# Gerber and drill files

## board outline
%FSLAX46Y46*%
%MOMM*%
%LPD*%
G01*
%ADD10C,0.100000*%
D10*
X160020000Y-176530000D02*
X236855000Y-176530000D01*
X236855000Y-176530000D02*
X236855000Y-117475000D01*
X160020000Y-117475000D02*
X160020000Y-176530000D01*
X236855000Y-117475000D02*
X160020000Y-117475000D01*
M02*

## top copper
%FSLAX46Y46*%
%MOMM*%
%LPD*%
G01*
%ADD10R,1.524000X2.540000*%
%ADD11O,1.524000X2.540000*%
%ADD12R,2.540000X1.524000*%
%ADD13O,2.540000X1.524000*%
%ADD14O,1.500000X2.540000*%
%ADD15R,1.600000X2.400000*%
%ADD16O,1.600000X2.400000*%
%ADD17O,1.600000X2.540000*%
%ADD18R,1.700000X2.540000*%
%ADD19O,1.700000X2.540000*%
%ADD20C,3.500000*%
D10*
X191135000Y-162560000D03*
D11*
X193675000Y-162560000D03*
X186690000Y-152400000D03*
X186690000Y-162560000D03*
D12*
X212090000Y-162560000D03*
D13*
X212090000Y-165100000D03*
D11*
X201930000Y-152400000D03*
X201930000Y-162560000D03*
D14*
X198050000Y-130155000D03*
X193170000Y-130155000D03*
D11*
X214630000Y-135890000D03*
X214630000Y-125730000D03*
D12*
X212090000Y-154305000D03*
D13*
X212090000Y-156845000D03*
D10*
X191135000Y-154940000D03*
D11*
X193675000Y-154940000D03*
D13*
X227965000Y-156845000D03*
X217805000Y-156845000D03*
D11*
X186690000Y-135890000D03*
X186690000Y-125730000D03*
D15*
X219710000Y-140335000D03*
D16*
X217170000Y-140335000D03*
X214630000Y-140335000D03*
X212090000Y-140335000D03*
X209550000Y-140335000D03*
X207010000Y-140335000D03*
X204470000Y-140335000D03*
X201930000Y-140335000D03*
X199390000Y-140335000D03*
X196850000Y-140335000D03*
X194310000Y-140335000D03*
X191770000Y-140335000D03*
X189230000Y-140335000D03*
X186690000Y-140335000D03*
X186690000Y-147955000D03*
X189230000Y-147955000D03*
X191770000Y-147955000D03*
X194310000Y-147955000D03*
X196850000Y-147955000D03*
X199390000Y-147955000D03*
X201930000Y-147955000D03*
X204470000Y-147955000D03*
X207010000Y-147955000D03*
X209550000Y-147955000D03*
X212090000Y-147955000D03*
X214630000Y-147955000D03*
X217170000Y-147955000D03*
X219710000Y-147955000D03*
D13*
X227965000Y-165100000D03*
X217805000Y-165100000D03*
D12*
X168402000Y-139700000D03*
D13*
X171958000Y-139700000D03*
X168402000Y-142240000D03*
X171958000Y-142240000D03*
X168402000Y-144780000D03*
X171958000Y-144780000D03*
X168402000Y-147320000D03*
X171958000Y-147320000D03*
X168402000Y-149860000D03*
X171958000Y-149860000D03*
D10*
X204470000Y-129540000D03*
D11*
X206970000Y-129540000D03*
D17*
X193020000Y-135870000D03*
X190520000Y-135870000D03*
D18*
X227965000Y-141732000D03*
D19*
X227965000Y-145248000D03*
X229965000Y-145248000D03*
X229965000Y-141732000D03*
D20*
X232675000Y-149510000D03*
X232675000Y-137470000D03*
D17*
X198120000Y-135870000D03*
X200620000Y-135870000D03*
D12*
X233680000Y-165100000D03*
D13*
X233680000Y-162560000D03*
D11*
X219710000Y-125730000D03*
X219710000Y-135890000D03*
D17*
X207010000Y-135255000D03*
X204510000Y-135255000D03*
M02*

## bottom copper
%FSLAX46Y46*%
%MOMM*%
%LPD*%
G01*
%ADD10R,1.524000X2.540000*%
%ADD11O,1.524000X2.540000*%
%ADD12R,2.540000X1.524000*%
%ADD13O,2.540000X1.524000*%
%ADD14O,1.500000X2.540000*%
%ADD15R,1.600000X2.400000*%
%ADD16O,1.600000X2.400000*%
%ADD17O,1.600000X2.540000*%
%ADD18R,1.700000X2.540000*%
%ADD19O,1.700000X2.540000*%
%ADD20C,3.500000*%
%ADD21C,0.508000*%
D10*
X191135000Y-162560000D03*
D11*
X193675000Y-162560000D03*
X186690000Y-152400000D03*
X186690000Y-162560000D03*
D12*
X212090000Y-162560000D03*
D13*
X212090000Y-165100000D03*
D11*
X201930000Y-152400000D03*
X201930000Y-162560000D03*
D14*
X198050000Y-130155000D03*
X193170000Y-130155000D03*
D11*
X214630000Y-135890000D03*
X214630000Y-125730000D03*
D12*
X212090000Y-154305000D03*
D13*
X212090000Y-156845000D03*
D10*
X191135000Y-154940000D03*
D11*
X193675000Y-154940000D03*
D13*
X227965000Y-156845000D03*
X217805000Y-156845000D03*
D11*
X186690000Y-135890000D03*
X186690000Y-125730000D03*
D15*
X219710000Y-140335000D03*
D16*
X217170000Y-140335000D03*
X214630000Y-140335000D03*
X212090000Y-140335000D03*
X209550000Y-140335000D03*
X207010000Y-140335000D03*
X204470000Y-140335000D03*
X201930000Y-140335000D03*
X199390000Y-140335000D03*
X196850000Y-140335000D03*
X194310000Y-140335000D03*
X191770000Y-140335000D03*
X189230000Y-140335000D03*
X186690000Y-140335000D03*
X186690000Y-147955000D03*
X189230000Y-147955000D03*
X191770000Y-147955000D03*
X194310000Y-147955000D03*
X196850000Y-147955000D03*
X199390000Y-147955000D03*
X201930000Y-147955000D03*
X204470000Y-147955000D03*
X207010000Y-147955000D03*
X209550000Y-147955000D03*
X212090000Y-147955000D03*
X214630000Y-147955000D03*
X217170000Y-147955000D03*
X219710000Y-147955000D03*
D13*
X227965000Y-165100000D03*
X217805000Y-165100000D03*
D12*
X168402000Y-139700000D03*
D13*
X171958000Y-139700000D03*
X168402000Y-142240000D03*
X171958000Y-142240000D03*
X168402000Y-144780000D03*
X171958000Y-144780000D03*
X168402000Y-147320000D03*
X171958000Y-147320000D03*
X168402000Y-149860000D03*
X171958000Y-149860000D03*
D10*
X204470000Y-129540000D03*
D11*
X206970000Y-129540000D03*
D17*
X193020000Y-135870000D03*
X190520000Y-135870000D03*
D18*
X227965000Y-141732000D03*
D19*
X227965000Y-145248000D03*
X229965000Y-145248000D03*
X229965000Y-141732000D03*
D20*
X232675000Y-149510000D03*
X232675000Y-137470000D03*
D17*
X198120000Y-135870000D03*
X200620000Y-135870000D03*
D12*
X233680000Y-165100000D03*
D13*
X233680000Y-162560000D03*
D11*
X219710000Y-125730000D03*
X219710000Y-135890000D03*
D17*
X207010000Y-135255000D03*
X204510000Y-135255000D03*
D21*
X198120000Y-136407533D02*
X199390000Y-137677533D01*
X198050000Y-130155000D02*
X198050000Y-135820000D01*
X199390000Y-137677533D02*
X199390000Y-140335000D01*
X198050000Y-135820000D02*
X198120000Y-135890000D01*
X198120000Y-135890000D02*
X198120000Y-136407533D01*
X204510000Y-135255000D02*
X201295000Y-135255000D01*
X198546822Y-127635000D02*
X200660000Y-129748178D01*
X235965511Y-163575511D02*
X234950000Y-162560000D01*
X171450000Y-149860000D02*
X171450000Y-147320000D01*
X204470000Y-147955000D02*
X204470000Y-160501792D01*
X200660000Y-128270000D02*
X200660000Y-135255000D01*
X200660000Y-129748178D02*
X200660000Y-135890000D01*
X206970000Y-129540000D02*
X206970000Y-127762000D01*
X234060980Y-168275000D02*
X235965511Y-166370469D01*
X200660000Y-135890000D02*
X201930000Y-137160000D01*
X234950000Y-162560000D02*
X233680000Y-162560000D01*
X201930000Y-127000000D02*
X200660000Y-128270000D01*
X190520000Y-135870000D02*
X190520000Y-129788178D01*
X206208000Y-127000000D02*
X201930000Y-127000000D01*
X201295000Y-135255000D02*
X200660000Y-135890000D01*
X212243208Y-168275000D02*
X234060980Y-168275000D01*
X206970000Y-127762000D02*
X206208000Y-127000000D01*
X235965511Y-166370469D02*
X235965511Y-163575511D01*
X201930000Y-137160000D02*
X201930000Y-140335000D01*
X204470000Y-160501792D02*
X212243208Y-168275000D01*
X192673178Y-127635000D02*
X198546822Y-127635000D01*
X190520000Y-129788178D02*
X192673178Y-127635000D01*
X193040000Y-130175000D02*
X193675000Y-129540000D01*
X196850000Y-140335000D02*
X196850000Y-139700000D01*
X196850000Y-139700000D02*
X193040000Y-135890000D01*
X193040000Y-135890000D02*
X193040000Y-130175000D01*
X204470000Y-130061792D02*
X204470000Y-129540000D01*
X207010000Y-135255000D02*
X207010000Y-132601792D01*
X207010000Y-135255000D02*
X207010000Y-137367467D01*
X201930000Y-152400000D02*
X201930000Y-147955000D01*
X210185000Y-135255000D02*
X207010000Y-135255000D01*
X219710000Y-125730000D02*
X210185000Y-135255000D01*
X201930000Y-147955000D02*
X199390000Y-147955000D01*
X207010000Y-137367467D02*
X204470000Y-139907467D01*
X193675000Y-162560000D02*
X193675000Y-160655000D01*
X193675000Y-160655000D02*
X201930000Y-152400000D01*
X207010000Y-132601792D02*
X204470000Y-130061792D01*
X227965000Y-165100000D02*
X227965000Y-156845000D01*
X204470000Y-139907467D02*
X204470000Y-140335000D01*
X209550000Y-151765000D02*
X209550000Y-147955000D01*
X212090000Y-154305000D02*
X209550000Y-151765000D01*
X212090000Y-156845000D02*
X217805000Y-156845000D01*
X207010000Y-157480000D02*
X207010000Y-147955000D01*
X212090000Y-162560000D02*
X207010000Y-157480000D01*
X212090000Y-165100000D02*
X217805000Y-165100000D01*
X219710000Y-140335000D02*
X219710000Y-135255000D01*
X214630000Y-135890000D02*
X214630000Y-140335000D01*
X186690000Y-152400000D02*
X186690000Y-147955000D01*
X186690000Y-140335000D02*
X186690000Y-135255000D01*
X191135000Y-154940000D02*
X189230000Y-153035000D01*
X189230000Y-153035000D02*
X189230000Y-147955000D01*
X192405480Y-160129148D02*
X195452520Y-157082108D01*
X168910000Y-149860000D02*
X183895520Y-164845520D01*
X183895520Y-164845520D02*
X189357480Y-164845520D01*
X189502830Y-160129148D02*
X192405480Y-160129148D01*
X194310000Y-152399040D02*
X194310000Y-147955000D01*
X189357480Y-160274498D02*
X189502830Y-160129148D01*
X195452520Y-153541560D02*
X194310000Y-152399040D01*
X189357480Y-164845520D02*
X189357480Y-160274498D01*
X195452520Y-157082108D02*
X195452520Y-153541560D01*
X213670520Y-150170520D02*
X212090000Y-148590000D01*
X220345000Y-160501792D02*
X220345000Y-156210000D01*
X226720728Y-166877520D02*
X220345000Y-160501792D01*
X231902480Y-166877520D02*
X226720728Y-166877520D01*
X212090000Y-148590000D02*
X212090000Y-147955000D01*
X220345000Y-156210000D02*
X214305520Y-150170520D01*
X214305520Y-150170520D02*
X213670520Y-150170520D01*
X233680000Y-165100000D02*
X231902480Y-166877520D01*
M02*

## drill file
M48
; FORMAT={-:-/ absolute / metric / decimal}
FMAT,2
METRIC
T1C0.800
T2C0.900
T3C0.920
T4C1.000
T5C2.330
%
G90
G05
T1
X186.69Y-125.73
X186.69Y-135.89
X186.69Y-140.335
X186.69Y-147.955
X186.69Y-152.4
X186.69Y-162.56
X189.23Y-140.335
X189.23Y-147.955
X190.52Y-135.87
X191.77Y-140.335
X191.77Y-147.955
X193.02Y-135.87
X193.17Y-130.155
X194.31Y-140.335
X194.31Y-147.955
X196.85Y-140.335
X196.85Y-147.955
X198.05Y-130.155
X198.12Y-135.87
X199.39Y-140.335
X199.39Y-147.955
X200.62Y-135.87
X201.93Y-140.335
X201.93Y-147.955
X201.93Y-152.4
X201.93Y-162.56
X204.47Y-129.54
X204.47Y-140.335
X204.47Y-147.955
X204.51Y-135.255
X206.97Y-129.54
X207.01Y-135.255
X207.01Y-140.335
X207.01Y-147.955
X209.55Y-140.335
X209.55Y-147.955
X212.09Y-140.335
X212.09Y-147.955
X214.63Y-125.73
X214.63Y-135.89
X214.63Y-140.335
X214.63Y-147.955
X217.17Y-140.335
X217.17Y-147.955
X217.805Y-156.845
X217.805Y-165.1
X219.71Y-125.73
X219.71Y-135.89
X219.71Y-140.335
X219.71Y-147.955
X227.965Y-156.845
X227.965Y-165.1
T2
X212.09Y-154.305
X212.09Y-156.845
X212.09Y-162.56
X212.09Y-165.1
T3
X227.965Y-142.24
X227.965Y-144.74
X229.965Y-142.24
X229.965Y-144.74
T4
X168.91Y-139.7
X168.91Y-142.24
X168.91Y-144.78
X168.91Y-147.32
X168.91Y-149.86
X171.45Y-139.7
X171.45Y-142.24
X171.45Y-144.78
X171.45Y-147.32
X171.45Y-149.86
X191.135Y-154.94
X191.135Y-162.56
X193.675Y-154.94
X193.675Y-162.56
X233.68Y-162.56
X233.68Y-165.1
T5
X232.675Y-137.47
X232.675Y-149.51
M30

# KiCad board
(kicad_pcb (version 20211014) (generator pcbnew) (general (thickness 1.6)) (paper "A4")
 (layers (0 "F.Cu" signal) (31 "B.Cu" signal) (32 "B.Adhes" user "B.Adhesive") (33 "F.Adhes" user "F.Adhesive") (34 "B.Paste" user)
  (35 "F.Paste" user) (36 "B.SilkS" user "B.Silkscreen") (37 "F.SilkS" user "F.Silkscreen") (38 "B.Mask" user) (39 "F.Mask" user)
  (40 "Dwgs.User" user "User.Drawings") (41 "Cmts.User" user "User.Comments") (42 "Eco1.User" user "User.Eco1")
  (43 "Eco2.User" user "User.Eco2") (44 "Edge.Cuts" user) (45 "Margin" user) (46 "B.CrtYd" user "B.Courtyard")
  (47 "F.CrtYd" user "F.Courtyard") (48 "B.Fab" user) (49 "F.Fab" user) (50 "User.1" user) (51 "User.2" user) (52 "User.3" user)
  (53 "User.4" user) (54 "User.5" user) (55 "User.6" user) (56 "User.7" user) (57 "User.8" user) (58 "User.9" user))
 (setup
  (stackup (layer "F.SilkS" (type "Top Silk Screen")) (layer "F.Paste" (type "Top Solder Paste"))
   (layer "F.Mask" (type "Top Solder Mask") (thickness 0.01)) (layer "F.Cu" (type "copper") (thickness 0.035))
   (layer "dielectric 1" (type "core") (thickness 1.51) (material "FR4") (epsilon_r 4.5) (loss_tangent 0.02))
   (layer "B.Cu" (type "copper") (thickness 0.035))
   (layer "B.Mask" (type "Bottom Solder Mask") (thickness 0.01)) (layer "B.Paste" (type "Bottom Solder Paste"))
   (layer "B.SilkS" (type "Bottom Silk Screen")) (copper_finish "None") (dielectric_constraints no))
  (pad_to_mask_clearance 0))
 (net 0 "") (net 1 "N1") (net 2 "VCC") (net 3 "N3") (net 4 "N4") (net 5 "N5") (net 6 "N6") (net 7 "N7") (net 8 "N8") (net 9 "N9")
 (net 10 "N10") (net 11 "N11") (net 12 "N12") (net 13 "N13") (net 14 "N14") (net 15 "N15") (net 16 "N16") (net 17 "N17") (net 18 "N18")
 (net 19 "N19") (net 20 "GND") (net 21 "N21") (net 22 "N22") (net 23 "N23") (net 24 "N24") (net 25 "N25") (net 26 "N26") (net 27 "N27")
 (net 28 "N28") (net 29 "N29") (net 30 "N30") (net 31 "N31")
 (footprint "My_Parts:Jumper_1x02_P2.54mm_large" (layer "F.Cu") (at 191.135 162.56 90)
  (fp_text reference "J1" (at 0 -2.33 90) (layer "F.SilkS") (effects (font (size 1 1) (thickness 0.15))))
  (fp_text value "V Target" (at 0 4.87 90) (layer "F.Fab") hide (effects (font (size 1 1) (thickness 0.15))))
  (pad "1" thru_hole rect locked (at 0 0 90) (size 2.54 1.524) (drill 1) (layers *.Cu *.Mask) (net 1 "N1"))
  (pad "2" thru_hole oval locked (at 0 2.54 90) (size 2.54 1.524) (drill 1) (layers *.Cu *.Mask) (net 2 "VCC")))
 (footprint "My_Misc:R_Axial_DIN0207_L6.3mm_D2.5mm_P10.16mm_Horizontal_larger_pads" (layer "F.Cu") (at 186.69 152.4 -90)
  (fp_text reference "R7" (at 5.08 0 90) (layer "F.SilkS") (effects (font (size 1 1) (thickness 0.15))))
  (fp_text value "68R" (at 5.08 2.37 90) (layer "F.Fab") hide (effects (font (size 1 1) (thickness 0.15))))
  (pad "1" thru_hole oval (at 0 0 270) (size 2.54 1.524) (drill 0.8) (layers *.Cu *.Mask) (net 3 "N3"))
  (pad "2" thru_hole oval (at 10.16 0 270) (size 2.54 1.524) (drill 0.8) (layers *.Cu *.Mask) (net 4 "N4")))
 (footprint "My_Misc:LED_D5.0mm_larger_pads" (layer "F.Cu") (at 212.09 162.56 -90)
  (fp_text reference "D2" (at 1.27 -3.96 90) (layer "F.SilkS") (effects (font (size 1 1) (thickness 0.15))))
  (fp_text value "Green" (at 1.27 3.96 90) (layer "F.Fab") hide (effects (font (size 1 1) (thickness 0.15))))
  (pad "1" thru_hole rect locked (at 0 0 270) (size 1.524 2.54) (drill 0.9) (layers *.Cu *.Mask) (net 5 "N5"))
  (pad "2" thru_hole oval locked (at 2.54 0 270) (size 1.524 2.54) (drill 0.9) (layers *.Cu *.Mask) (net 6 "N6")))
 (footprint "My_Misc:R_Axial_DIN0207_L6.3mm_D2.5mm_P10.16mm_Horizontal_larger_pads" (layer "F.Cu") (at 201.93 152.4 -90)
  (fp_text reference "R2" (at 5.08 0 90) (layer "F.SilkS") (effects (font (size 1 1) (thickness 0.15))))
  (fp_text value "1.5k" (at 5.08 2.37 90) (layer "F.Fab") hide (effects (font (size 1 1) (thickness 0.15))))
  (pad "1" thru_hole oval (at 0 0 270) (size 2.54 1.524) (drill 0.8) (layers *.Cu *.Mask) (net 2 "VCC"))
  (pad "2" thru_hole oval (at 10.16 0 270) (size 2.54 1.524) (drill 0.8) (layers *.Cu *.Mask) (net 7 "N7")))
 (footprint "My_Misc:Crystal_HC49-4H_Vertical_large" (layer "F.Cu") (at 198.05 130.155 180)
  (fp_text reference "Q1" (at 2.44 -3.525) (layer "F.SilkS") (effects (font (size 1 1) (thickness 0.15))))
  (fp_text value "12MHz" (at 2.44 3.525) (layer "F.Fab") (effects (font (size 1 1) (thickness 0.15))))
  (pad "1" thru_hole oval locked (at 0 0 180) (size 1.5 2.54) (drill 0.8) (layers *.Cu *.Mask) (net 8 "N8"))
  (pad "2" thru_hole oval locked (at 4.88 0 180) (size 1.5 2.54) (drill 0.8) (layers *.Cu *.Mask) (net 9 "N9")))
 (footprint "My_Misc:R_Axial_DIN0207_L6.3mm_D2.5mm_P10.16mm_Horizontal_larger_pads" (layer "F.Cu") (at 214.63 135.89 90)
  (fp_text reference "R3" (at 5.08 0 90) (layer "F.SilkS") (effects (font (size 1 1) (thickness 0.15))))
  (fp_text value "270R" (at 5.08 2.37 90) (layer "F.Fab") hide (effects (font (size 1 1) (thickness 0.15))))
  (pad "1" thru_hole oval (at 0 0 90) (size 2.54 1.524) (drill 0.8) (layers *.Cu *.Mask) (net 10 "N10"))
  (pad "2" thru_hole oval (at 10.16 0 90) (size 2.54 1.524) (drill 0.8) (layers *.Cu *.Mask) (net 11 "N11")))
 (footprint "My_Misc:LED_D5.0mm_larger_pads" (layer "F.Cu") (at 212.09 154.305 -90)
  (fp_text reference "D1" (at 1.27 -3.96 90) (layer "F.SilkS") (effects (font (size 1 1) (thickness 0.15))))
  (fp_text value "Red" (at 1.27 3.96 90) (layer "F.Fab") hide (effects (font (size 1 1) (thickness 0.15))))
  (pad "1" thru_hole rect locked (at 0 0 270) (size 1.524 2.54) (drill 0.9) (layers *.Cu *.Mask) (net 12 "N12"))
  (pad "2" thru_hole oval locked (at 2.54 0 270) (size 1.524 2.54) (drill 0.9) (layers *.Cu *.Mask) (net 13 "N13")))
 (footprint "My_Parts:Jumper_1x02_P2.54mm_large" (layer "F.Cu") (at 191.135 154.94 90)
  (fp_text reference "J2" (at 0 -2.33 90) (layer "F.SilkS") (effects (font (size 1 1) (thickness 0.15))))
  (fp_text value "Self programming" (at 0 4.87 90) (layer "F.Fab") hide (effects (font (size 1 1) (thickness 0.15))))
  (pad "1" thru_hole rect locked (at 0 0 90) (size 2.54 1.524) (drill 1) (layers *.Cu *.Mask) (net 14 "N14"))
  (pad "2" thru_hole oval locked (at 0 2.54 90) (size 2.54 1.524) (drill 1) (layers *.Cu *.Mask) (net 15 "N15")))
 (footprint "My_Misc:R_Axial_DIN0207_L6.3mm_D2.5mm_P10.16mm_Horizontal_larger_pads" (layer "F.Cu") (at 227.965 156.845 180)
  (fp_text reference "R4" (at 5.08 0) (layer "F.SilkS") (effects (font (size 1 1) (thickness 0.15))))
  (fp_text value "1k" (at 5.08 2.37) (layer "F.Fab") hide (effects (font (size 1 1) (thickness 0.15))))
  (pad "1" thru_hole oval (at 0 0 180) (size 2.54 1.524) (drill 0.8) (layers *.Cu *.Mask) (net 2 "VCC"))
  (pad "2" thru_hole oval (at 10.16 0 180) (size 2.54 1.524) (drill 0.8) (layers *.Cu *.Mask) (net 13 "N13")))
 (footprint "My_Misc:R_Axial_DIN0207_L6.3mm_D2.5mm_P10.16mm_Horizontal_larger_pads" (layer "F.Cu") (at 186.69 135.89 90)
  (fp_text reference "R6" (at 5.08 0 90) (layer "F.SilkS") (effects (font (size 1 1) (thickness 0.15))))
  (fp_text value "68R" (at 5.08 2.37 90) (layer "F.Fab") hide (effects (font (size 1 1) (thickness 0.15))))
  (pad "1" thru_hole oval (at 0 0 90) (size 2.54 1.524) (drill 0.8) (layers *.Cu *.Mask) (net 7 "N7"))
  (pad "2" thru_hole oval (at 10.16 0 90) (size 2.54 1.524) (drill 0.8) (layers *.Cu *.Mask) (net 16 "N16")))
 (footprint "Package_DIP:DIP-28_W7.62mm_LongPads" (layer "F.Cu") (at 219.71 140.335 -90)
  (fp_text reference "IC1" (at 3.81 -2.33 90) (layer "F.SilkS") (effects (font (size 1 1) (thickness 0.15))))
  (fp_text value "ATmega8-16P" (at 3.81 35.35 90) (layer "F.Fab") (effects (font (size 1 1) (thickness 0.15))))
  (pad "1" thru_hole rect (at 0 0 270) (size 2.4 1.6) (drill 0.8) (layers *.Cu *.Mask) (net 15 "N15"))
  (pad "2" thru_hole oval (at 0 2.54 270) (size 2.4 1.6) (drill 0.8) (layers *.Cu *.Mask) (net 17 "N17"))
  (pad "3" thru_hole oval (at 0 5.08 270) (size 2.4 1.6) (drill 0.8) (layers *.Cu *.Mask) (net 10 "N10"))
  (pad "4" thru_hole oval (at 0 7.62 270) (size 2.4 1.6) (drill 0.8) (layers *.Cu *.Mask) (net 3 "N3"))
  (pad "5" thru_hole oval (at 0 10.16 270) (size 2.4 1.6) (drill 0.8) (layers *.Cu *.Mask) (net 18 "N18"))
  (pad "6" thru_hole oval (at 0 12.7 270) (size 2.4 1.6) (drill 0.8) (layers *.Cu *.Mask) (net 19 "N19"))
  (pad "7" thru_hole oval (at 0 15.24 270) (size 2.4 1.6) (drill 0.8) (layers *.Cu *.Mask) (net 2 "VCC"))
  (pad "8" thru_hole oval (at 0 17.78 270) (size 2.4 1.6) (drill 0.8) (layers *.Cu *.Mask) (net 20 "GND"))
  (pad "9" thru_hole oval (at 0 20.32 270) (size 2.4 1.6) (drill 0.8) (layers *.Cu *.Mask) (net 8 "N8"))
  (pad "10" thru_hole oval (at 0 22.86 270) (size 2.4 1.6) (drill 0.8) (layers *.Cu *.Mask) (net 9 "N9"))
  (pad "11" thru_hole oval (at 0 25.4 270) (size 2.4 1.6) (drill 0.8) (layers *.Cu *.Mask) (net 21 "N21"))
  (pad "12" thru_hole oval (at 0 27.94 270) (size 2.4 1.6) (drill 0.8) (layers *.Cu *.Mask) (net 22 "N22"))
  (pad "13" thru_hole oval (at 0 30.48 270) (size 2.4 1.6) (drill 0.8) (layers *.Cu *.Mask) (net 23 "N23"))
  (pad "14" thru_hole oval (at 0 33.02 270) (size 2.4 1.6) (drill 0.8) (layers *.Cu *.Mask) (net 7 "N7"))
  (pad "15" thru_hole oval (at 7.62 33.02 270) (size 2.4 1.6) (drill 0.8) (layers *.Cu *.Mask) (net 3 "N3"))
  (pad "16" thru_hole oval (at 7.62 30.48 270) (size 2.4 1.6) (drill 0.8) (layers *.Cu *.Mask) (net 14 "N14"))
  (pad "17" thru_hole oval (at 7.62 27.94 270) (size 2.4 1.6) (drill 0.8) (layers *.Cu *.Mask) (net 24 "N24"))
  (pad "18" thru_hole oval (at 7.62 25.4 270) (size 2.4 1.6) (drill 0.8) (layers *.Cu *.Mask) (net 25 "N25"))
  (pad "19" thru_hole oval (at 7.62 22.86 270) (size 2.4 1.6) (drill 0.8) (layers *.Cu *.Mask) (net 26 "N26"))
  (pad "20" thru_hole oval (at 7.62 20.32 270) (size 2.4 1.6) (drill 0.8) (layers *.Cu *.Mask) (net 2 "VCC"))
  (pad "21" thru_hole oval (at 7.62 17.78 270) (size 2.4 1.6) (drill 0.8) (layers *.Cu *.Mask) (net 2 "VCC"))
  (pad "22" thru_hole oval (at 7.62 15.24 270) (size 2.4 1.6) (drill 0.8) (layers *.Cu *.Mask) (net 20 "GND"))
  (pad "23" thru_hole oval (at 7.62 12.7 270) (size 2.4 1.6) (drill 0.8) (layers *.Cu *.Mask) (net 5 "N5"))
  (pad "24" thru_hole oval (at 7.62 10.16 270) (size 2.4 1.6) (drill 0.8) (layers *.Cu *.Mask) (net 12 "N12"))
  (pad "25" thru_hole oval (at 7.62 7.62 270) (size 2.4 1.6) (drill 0.8) (layers *.Cu *.Mask) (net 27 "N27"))
  (pad "26" thru_hole oval (at 7.62 5.08 270) (size 2.4 1.6) (drill 0.8) (layers *.Cu *.Mask) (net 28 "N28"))
  (pad "27" thru_hole oval (at 7.62 2.54 270) (size 2.4 1.6) (drill 0.8) (layers *.Cu *.Mask) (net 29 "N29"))
  (pad "28" thru_hole oval (at 7.62 0 270) (size 2.4 1.6) (drill 0.8) (layers *.Cu *.Mask) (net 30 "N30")))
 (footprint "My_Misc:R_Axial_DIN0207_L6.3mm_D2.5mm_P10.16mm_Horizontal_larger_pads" (layer "F.Cu") (at 227.965 165.1 180)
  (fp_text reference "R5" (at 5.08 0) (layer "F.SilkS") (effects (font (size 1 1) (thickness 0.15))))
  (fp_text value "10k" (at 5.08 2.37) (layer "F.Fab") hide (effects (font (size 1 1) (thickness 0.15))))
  (pad "1" thru_hole oval (at 0 0 180) (size 2.54 1.524) (drill 0.8) (layers *.Cu *.Mask) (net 2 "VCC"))
  (pad "2" thru_hole oval (at 10.16 0 180) (size 2.54 1.524) (drill 0.8) (layers *.Cu *.Mask) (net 6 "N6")))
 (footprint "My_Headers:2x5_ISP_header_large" (layer "F.Cu") (at 168.91 139.7)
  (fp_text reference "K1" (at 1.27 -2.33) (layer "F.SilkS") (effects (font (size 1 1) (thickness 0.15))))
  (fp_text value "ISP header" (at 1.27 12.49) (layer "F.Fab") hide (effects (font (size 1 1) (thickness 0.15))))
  (pad "1" thru_hole rect locked (at 0 0) (size 2.54 1.524) (drill 1 (offset -0.508 0)) (layers *.Cu *.Mask) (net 24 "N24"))
  (pad "2" thru_hole oval locked (at 2.54 0) (size 2.54 1.524) (drill 1 (offset 0.508 0)) (layers *.Cu *.Mask) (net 1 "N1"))
  (pad "3" thru_hole oval locked (at 0 2.54) (size 2.54 1.524) (drill 1 (offset -0.508 0)) (layers *.Cu *.Mask) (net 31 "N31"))
  (pad "4" thru_hole oval locked (at 2.54 2.54) (size 2.54 1.524) (drill 1 (offset 0.508 0)) (layers *.Cu *.Mask) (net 11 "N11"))
  (pad "5" thru_hole oval locked (at 0 5.08) (size 2.54 1.524) (drill 1 (offset -0.508 0)) (layers *.Cu *.Mask) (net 14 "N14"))
  (pad "6" thru_hole oval locked (at 2.54 5.08) (size 2.54 1.524) (drill 1 (offset 0.508 0)) (layers *.Cu *.Mask) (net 17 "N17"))
  (pad "7" thru_hole oval locked (at 0 7.62) (size 2.54 1.524) (drill 1 (offset -0.508 0)) (layers *.Cu *.Mask) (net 26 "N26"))
  (pad "8" thru_hole oval locked (at 2.54 7.62) (size 2.54 1.524) (drill 1 (offset 0.508 0)) (layers *.Cu *.Mask) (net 20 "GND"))
  (pad "9" thru_hole oval locked (at 0 10.16) (size 2.54 1.524) (drill 1 (offset -0.508 0)) (layers *.Cu *.Mask) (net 25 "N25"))
  (pad "10" thru_hole oval locked (at 2.54 10.16) (size 2.54 1.524) (drill 1 (offset 0.508 0)) (layers *.Cu *.Mask) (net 20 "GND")))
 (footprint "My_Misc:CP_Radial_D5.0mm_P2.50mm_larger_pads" (layer "F.Cu") (at 204.47 129.54)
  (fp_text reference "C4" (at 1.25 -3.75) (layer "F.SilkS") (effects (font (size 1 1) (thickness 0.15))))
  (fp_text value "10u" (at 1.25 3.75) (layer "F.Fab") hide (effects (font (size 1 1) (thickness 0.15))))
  (pad "1" thru_hole rect (at 0 0) (size 1.524 2.54) (drill 0.8) (layers *.Cu *.Mask) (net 2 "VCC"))
  (pad "2" thru_hole oval (at 2.5 0) (size 1.524 2.54) (drill 0.8) (layers *.Cu *.Mask) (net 20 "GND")))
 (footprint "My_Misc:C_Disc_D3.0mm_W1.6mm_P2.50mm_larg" (layer "F.Cu") (at 193.02 135.87 180)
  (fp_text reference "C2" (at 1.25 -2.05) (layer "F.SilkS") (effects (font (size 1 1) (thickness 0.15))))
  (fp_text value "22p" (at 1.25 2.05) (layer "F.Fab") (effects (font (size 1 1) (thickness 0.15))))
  (pad "1" thru_hole oval locked (at 0 0 180) (size 1.6 2.54) (drill 0.8) (layers *.Cu *.Mask) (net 9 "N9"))
  (pad "2" thru_hole oval locked (at 2.5 0 180) (size 1.6 2.54) (drill 0.8) (layers *.Cu *.Mask) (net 20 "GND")))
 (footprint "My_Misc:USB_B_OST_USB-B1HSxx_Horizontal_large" (layer "F.Cu") (at 227.965 142.24)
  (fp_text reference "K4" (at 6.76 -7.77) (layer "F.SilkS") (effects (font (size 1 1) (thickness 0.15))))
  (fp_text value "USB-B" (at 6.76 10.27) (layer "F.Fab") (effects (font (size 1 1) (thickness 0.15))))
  (pad "1" thru_hole rect locked (at 0 0) (size 1.7 2.54) (drill 0.92 (offset 0 -0.508)) (layers *.Cu *.Mask) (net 2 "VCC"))
  (pad "2" thru_hole oval locked (at 0 2.5) (size 1.7 2.54) (drill 0.92 (offset 0 0.508)) (layers *.Cu *.Mask) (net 16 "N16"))
  (pad "3" thru_hole oval locked (at 2 2.5) (size 1.7 2.54) (drill 0.92 (offset 0 0.508)) (layers *.Cu *.Mask) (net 4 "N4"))
  (pad "4" thru_hole oval locked (at 2 0) (size 1.7 2.54) (drill 0.92 (offset 0 -0.508)) (layers *.Cu *.Mask) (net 20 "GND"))
  (pad "5" thru_hole circle locked (at 4.71 7.27) (size 3.5 3.5) (drill 2.33) (layers *.Cu *.Mask) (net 20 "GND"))
  (pad "5" thru_hole circle locked (at 4.71 -4.77) (size 3.5 3.5) (drill 2.33) (layers *.Cu *.Mask) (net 20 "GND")))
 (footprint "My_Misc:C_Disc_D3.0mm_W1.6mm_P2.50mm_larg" (layer "F.Cu") (at 198.12 135.87)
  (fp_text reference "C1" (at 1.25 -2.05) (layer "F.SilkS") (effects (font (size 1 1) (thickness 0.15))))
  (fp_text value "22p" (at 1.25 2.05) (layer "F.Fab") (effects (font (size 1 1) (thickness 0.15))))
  (pad "1" thru_hole oval locked (at 0 0) (size 1.6 2.54) (drill 0.8) (layers *.Cu *.Mask) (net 8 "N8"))
  (pad "2" thru_hole oval locked (at 2.5 0) (size 1.6 2.54) (drill 0.8) (layers *.Cu *.Mask) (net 20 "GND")))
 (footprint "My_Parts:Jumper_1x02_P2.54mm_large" (layer "F.Cu") (at 233.68 165.1 180)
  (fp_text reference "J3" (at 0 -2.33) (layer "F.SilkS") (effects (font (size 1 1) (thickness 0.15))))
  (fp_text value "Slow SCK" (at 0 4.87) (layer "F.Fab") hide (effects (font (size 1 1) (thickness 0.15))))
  (pad "1" thru_hole rect locked (at 0 0 180) (size 2.54 1.524) (drill 1) (layers *.Cu *.Mask) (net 27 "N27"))
  (pad "2" thru_hole oval locked (at 0 2.54 180) (size 2.54 1.524) (drill 1) (layers *.Cu *.Mask) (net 20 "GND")))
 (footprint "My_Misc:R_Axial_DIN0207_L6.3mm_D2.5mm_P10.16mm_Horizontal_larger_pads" (layer "F.Cu") (at 219.71 125.73 -90)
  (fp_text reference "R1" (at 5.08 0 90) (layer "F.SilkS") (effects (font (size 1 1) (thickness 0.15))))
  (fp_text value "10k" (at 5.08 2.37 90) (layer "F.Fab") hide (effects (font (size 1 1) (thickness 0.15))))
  (pad "1" thru_hole oval (at 0 0 270) (size 2.54 1.524) (drill 0.8) (layers *.Cu *.Mask) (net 2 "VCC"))
  (pad "2" thru_hole oval (at 10.16 0 270) (size 2.54 1.524) (drill 0.8) (layers *.Cu *.Mask) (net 15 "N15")))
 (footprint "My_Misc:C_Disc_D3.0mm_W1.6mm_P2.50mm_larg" (layer "F.Cu") (at 207.01 135.255 180)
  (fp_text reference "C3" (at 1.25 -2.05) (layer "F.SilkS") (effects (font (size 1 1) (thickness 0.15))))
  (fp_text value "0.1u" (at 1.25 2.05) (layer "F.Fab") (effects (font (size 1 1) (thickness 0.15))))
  (pad "1" thru_hole oval locked (at 0 0 180) (size 1.6 2.54) (drill 0.8) (layers *.Cu *.Mask) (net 2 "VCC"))
  (pad "2" thru_hole oval locked (at 2.5 0 180) (size 1.6 2.54) (drill 0.8) (layers *.Cu *.Mask) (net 20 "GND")))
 (gr_line (start 160.02 176.53) (end 236.855 176.53) (layer "Edge.Cuts") (width 0.1))
 (gr_line (start 236.855 176.53) (end 236.855 117.475) (layer "Edge.Cuts") (width 0.1))
 (gr_line (start 160.02 117.475) (end 160.02 176.53) (layer "Edge.Cuts") (width 0.1))
 (gr_line (start 236.855 117.475) (end 160.02 117.475) (layer "Edge.Cuts") (width 0.1))
 (segment (start 198.12 136.407533) (end 199.39 137.677533) (width 0.508) (layer "B.Cu") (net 8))
 (segment (start 198.05 130.155) (end 198.05 135.82) (width 0.508) (layer "B.Cu") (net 8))
 (segment (start 199.39 137.677533) (end 199.39 140.335) (width 0.508) (layer "B.Cu") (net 8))
 (segment (start 198.05 135.82) (end 198.12 135.89) (width 0.508) (layer "B.Cu") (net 8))
 (segment (start 198.12 135.89) (end 198.12 136.407533) (width 0.508) (layer "B.Cu") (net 8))
 (segment (start 204.51 135.255) (end 201.295 135.255) (width 0.508) (layer "B.Cu") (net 20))
 (segment (start 198.546822 127.635) (end 200.66 129.748178) (width 0.508) (layer "B.Cu") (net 20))
 (segment (start 235.965511 163.575511) (end 234.95 162.56) (width 0.508) (layer "B.Cu") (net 20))
 (segment (start 171.45 149.86) (end 171.45 147.32) (width 0.508) (layer "B.Cu") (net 20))
 (segment (start 204.47 147.955) (end 204.47 160.501792) (width 0.508) (layer "B.Cu") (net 20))
 (segment (start 200.66 128.27) (end 200.66 135.255) (width 0.508) (layer "B.Cu") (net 20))
 (segment (start 200.66 129.748178) (end 200.66 135.89) (width 0.508) (layer "B.Cu") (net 20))
 (segment (start 206.97 129.54) (end 206.97 127.762) (width 0.508) (layer "B.Cu") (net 20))
 (segment (start 234.06098 168.275) (end 235.965511 166.370469) (width 0.508) (layer "B.Cu") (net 20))
 (segment (start 200.66 135.89) (end 201.93 137.16) (width 0.508) (layer "B.Cu") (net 20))
 (segment (start 234.95 162.56) (end 233.68 162.56) (width 0.508) (layer "B.Cu") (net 20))
 (segment (start 201.93 127) (end 200.66 128.27) (width 0.508) (layer "B.Cu") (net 20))
 (segment (start 190.52 135.87) (end 190.52 129.788178) (width 0.508) (layer "B.Cu") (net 20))
 (segment (start 206.208 127) (end 201.93 127) (width 0.508) (layer "B.Cu") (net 20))
 (segment (start 201.295 135.255) (end 200.66 135.89) (width 0.508) (layer "B.Cu") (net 20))
 (segment (start 212.243208 168.275) (end 234.06098 168.275) (width 0.508) (layer "B.Cu") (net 20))
 (segment (start 206.97 127.762) (end 206.208 127) (width 0.508) (layer "B.Cu") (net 20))
 (segment (start 235.965511 166.370469) (end 235.965511 163.575511) (width 0.508) (layer "B.Cu") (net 20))
 (segment (start 201.93 137.16) (end 201.93 140.335) (width 0.508) (layer "B.Cu") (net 20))
 (segment (start 204.47 160.501792) (end 212.243208 168.275) (width 0.508) (layer "B.Cu") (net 20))
 (segment (start 192.673178 127.635) (end 198.546822 127.635) (width 0.508) (layer "B.Cu") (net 20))
 (segment (start 190.52 129.788178) (end 192.673178 127.635) (width 0.508) (layer "B.Cu") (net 20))
 (segment (start 193.04 130.175) (end 193.675 129.54) (width 0.508) (layer "B.Cu") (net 9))
 (segment (start 196.85 140.335) (end 196.85 139.7) (width 0.508) (layer "B.Cu") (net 9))
 (segment (start 196.85 139.7) (end 193.04 135.89) (width 0.508) (layer "B.Cu") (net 9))
 (segment (start 193.04 135.89) (end 193.04 130.175) (width 0.508) (layer "B.Cu") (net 9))
 (segment (start 204.47 130.061792) (end 204.47 129.54) (width 0.508) (layer "B.Cu") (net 2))
 (segment (start 207.01 135.255) (end 207.01 132.601792) (width 0.508) (layer "B.Cu") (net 2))
 (segment (start 207.01 135.255) (end 207.01 137.367467) (width 0.508) (layer "B.Cu") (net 2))
 (segment (start 201.93 152.4) (end 201.93 147.955) (width 0.508) (layer "B.Cu") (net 2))
 (segment (start 210.185 135.255) (end 207.01 135.255) (width 0.508) (layer "B.Cu") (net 2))
 (segment (start 219.71 125.73) (end 210.185 135.255) (width 0.508) (layer "B.Cu") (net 2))
 (segment (start 201.93 147.955) (end 199.39 147.955) (width 0.508) (layer "B.Cu") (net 2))
 (segment (start 207.01 137.367467) (end 204.47 139.907467) (width 0.508) (layer "B.Cu") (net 2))
 (segment (start 193.675 162.56) (end 193.675 160.655) (width 0.508) (layer "B.Cu") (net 2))
 (segment (start 193.675 160.655) (end 201.93 152.4) (width 0.508) (layer "B.Cu") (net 2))
 (segment (start 207.01 132.601792) (end 204.47 130.061792) (width 0.508) (layer "B.Cu") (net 2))
 (segment (start 227.965 165.1) (end 227.965 156.845) (width 0.508) (layer "B.Cu") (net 2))
 (segment (start 204.47 139.907467) (end 204.47 140.335) (width 0.508) (layer "B.Cu") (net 2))
 (segment (start 209.55 151.765) (end 209.55 147.955) (width 0.508) (layer "B.Cu") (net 12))
 (segment (start 212.09 154.305) (end 209.55 151.765) (width 0.508) (layer "B.Cu") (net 12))
 (segment (start 212.09 156.845) (end 217.805 156.845) (width 0.508) (layer "B.Cu") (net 13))
 (segment (start 207.01 157.48) (end 207.01 147.955) (width 0.508) (layer "B.Cu") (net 5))
 (segment (start 212.09 162.56) (end 207.01 157.48) (width 0.508) (layer "B.Cu") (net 5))
 (segment (start 212.09 165.1) (end 217.805 165.1) (width 0.508) (layer "B.Cu") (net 6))
 (segment (start 219.71 140.335) (end 219.71 135.255) (width 0.508) (layer "B.Cu") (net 15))
 (segment (start 214.63 135.89) (end 214.63 140.335) (width 0.508) (layer "B.Cu") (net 10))
 (segment (start 186.69 152.4) (end 186.69 147.955) (width 0.508) (layer "B.Cu") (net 3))
 (segment (start 186.69 140.335) (end 186.69 135.255) (width 0.508) (layer "B.Cu") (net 7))
 (segment (start 191.135 154.94) (end 189.23 153.035) (width 0.508) (layer "B.Cu") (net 14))
 (segment (start 189.23 153.035) (end 189.23 147.955) (width 0.508) (layer "B.Cu") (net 14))
 (segment (start 192.40548 160.129148) (end 195.45252 157.082108) (width 0.508) (layer "B.Cu") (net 25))
 (segment (start 168.91 149.86) (end 183.89552 164.84552) (width 0.508) (layer "B.Cu") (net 25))
 (segment (start 183.89552 164.84552) (end 189.35748 164.84552) (width 0.508) (layer "B.Cu") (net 25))
 (segment (start 189.50283 160.129148) (end 192.40548 160.129148) (width 0.508) (layer "B.Cu") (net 25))
 (segment (start 194.31 152.39904) (end 194.31 147.955) (width 0.508) (layer "B.Cu") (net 25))
 (segment (start 189.35748 160.274498) (end 189.50283 160.129148) (width 0.508) (layer "B.Cu") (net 25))
 (segment (start 195.45252 153.54156) (end 194.31 152.39904) (width 0.508) (layer "B.Cu") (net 25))
 (segment (start 189.35748 164.84552) (end 189.35748 160.274498) (width 0.508) (layer "B.Cu") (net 25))
 (segment (start 195.45252 157.082108) (end 195.45252 153.54156) (width 0.508) (layer "B.Cu") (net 25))
 (segment (start 213.67052 150.17052) (end 212.09 148.59) (width 0.508) (layer "B.Cu") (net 27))
 (segment (start 220.345 160.501792) (end 220.345 156.21) (width 0.508) (layer "B.Cu") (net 27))
 (segment (start 226.720728 166.87752) (end 220.345 160.501792) (width 0.508) (layer "B.Cu") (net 27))
 (segment (start 231.90248 166.87752) (end 226.720728 166.87752) (width 0.508) (layer "B.Cu") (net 27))
 (segment (start 212.09 148.59) (end 212.09 147.955) (width 0.508) (layer "B.Cu") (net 27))
 (segment (start 220.345 156.21) (end 214.30552 150.17052) (width 0.508) (layer "B.Cu") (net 27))
 (segment (start 214.30552 150.17052) (end 213.67052 150.17052) (width 0.508) (layer "B.Cu") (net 27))
 (segment (start 233.68 165.1) (end 231.90248 166.87752) (width 0.508) (layer "B.Cu") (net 27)))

